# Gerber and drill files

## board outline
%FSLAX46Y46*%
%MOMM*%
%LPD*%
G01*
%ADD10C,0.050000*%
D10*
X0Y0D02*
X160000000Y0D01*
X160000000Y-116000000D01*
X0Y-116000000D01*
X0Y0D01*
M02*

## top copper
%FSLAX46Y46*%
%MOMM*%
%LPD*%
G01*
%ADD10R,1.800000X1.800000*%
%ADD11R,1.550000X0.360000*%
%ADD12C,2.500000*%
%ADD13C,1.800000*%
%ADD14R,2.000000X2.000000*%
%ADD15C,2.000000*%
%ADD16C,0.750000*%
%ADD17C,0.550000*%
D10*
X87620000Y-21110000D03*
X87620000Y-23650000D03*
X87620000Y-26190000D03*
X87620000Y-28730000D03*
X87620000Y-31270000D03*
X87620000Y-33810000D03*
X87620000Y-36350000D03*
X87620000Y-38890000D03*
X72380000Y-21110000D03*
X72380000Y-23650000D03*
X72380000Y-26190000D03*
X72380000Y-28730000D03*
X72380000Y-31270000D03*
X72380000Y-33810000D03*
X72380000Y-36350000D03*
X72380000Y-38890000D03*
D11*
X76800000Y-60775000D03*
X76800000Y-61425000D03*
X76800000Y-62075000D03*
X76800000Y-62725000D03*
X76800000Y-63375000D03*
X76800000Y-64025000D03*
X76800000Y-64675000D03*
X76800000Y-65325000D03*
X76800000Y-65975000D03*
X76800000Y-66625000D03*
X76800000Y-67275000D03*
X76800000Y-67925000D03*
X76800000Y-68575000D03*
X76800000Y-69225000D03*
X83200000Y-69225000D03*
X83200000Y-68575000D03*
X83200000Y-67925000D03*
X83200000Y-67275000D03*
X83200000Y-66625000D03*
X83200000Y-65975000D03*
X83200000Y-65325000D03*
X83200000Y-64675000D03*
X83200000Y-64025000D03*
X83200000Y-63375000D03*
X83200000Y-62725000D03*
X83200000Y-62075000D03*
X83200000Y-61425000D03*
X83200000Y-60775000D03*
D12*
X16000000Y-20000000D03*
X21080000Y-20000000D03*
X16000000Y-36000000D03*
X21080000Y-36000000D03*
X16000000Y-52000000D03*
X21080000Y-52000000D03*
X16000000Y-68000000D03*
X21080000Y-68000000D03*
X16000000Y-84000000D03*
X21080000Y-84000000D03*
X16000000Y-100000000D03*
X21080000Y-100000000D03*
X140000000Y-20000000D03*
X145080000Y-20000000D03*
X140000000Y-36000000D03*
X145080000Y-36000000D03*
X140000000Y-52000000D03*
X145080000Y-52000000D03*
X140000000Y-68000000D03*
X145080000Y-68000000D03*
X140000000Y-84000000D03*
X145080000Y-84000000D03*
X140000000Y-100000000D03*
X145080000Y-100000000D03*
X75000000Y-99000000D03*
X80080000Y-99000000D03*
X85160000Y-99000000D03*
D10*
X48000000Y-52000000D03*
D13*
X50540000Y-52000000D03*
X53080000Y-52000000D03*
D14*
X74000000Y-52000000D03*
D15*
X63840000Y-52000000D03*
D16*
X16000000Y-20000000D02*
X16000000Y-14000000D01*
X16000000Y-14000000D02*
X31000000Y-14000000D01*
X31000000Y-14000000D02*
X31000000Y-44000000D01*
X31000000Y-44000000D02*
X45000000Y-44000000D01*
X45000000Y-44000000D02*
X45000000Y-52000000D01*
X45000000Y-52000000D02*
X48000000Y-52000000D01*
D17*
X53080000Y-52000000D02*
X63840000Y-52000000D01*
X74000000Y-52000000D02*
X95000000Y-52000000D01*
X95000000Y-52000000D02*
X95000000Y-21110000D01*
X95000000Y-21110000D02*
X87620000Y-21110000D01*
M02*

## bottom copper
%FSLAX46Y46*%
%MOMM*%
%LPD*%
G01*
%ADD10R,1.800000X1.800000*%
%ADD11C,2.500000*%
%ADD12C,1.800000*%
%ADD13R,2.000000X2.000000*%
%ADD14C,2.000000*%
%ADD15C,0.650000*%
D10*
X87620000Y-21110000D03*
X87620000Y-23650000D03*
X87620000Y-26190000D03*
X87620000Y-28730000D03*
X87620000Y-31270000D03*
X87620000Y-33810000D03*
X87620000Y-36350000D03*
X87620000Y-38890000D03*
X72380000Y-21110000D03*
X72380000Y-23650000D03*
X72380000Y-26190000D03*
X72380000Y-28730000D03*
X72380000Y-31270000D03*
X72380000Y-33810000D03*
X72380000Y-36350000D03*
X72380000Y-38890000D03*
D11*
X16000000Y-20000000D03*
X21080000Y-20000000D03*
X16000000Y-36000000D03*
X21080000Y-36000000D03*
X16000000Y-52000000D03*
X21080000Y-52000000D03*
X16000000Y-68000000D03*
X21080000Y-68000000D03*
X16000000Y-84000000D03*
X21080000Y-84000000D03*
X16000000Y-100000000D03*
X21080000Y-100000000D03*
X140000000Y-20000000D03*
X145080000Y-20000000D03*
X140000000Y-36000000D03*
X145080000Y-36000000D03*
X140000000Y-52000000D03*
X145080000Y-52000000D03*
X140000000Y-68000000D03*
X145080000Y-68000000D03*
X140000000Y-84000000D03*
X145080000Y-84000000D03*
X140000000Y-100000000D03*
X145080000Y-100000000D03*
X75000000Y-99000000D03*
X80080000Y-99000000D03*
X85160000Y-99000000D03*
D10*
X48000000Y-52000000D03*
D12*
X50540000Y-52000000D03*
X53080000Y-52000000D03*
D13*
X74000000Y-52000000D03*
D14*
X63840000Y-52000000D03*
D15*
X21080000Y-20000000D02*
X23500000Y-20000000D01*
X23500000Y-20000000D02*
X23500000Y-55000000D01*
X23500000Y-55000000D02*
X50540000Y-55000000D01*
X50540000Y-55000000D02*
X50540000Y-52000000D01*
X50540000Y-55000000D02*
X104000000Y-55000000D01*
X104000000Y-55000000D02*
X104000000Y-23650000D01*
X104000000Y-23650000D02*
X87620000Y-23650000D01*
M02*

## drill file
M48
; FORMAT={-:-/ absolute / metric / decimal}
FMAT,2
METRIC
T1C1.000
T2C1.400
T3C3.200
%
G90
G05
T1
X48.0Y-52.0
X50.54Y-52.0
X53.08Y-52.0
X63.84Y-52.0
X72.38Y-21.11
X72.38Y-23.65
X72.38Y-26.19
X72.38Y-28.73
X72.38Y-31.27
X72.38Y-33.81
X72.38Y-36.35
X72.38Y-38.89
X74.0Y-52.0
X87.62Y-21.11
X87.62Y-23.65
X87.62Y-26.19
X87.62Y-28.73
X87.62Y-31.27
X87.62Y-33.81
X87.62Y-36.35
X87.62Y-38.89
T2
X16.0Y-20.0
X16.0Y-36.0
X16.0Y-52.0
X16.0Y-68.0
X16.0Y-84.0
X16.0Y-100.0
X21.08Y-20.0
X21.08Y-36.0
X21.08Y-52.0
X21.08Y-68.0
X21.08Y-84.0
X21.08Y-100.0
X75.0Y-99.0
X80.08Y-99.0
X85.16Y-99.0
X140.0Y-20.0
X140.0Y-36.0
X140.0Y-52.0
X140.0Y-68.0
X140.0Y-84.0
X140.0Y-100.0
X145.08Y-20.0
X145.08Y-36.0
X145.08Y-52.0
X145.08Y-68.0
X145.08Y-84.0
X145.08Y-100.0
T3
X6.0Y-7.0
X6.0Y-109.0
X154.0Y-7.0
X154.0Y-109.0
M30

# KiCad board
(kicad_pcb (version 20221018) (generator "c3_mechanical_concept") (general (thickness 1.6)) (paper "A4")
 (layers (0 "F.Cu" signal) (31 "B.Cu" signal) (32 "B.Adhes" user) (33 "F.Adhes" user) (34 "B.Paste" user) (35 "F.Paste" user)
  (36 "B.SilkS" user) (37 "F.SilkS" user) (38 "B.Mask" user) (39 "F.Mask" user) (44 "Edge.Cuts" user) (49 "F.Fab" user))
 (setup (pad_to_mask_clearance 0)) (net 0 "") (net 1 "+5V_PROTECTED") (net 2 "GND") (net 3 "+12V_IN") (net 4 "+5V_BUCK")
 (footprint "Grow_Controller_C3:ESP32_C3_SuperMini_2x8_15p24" (layer "F.Cu") (at 80 30)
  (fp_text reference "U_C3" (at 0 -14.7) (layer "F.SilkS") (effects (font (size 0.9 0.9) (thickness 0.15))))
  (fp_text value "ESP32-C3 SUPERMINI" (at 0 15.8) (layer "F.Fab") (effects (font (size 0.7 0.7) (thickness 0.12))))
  (pad "1" thru_hole rect (at 7.62 -8.89) (size 1.8 1.8) (drill 1.0) (layers "*.Cu" "*.Mask") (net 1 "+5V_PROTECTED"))
  (pad "2" thru_hole rect (at 7.62 -6.35) (size 1.8 1.8) (drill 1.0) (layers "*.Cu" "*.Mask") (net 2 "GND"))
  (pad "3" thru_hole rect (at 7.62 -3.81) (size 1.8 1.8) (drill 1.0) (layers "*.Cu" "*.Mask"))
  (pad "4" thru_hole rect (at 7.62 -1.27) (size 1.8 1.8) (drill 1.0) (layers "*.Cu" "*.Mask"))
  (pad "5" thru_hole rect (at 7.62 1.27) (size 1.8 1.8) (drill 1.0) (layers "*.Cu" "*.Mask"))
  (pad "6" thru_hole rect (at 7.62 3.81) (size 1.8 1.8) (drill 1.0) (layers "*.Cu" "*.Mask"))
  (pad "7" thru_hole rect (at 7.62 6.35) (size 1.8 1.8) (drill 1.0) (layers "*.Cu" "*.Mask"))
  (pad "8" thru_hole rect (at 7.62 8.89) (size 1.8 1.8) (drill 1.0) (layers "*.Cu" "*.Mask"))
  (pad "9" thru_hole rect (at -7.62 -8.89) (size 1.8 1.8) (drill 1.0) (layers "*.Cu" "*.Mask"))
  (pad "10" thru_hole rect (at -7.62 -6.35) (size 1.8 1.8) (drill 1.0) (layers "*.Cu" "*.Mask"))
  (pad "11" thru_hole rect (at -7.62 -3.81) (size 1.8 1.8) (drill 1.0) (layers "*.Cu" "*.Mask"))
  (pad "12" thru_hole rect (at -7.62 -1.27) (size 1.8 1.8) (drill 1.0) (layers "*.Cu" "*.Mask"))
  (pad "13" thru_hole rect (at -7.62 1.27) (size 1.8 1.8) (drill 1.0) (layers "*.Cu" "*.Mask"))
  (pad "14" thru_hole rect (at -7.62 3.81) (size 1.8 1.8) (drill 1.0) (layers "*.Cu" "*.Mask"))
  (pad "15" thru_hole rect (at -7.62 6.35) (size 1.8 1.8) (drill 1.0) (layers "*.Cu" "*.Mask"))
  (pad "16" thru_hole rect (at -7.62 8.89) (size 1.8 1.8) (drill 1.0) (layers "*.Cu" "*.Mask")))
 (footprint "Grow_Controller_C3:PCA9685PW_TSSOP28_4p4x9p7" (layer "F.Cu") (at 80 65)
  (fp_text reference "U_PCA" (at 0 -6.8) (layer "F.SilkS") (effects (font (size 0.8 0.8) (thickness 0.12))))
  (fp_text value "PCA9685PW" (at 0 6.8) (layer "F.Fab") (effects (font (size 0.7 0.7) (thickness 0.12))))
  (pad "1" smd rect (at -3.200 -4.225) (size 1.55 0.36) (layers "F.Cu" "F.Paste" "F.Mask"))
  (pad "2" smd rect (at -3.200 -3.575) (size 1.55 0.36) (layers "F.Cu" "F.Paste" "F.Mask"))
  (pad "3" smd rect (at -3.200 -2.925) (size 1.55 0.36) (layers "F.Cu" "F.Paste" "F.Mask"))
  (pad "4" smd rect (at -3.200 -2.275) (size 1.55 0.36) (layers "F.Cu" "F.Paste" "F.Mask"))
  (pad "5" smd rect (at -3.200 -1.625) (size 1.55 0.36) (layers "F.Cu" "F.Paste" "F.Mask"))
  (pad "6" smd rect (at -3.200 -0.975) (size 1.55 0.36) (layers "F.Cu" "F.Paste" "F.Mask"))
  (pad "7" smd rect (at -3.200 -0.325) (size 1.55 0.36) (layers "F.Cu" "F.Paste" "F.Mask"))
  (pad "8" smd rect (at -3.200 0.325) (size 1.55 0.36) (layers "F.Cu" "F.Paste" "F.Mask"))
  (pad "9" smd rect (at -3.200 0.975) (size 1.55 0.36) (layers "F.Cu" "F.Paste" "F.Mask"))
  (pad "10" smd rect (at -3.200 1.625) (size 1.55 0.36) (layers "F.Cu" "F.Paste" "F.Mask"))
  (pad "11" smd rect (at -3.200 2.275) (size 1.55 0.36) (layers "F.Cu" "F.Paste" "F.Mask"))
  (pad "12" smd rect (at -3.200 2.925) (size 1.55 0.36) (layers "F.Cu" "F.Paste" "F.Mask"))
  (pad "13" smd rect (at -3.200 3.575) (size 1.55 0.36) (layers "F.Cu" "F.Paste" "F.Mask"))
  (pad "14" smd rect (at -3.200 4.225) (size 1.55 0.36) (layers "F.Cu" "F.Paste" "F.Mask"))
  (pad "15" smd rect (at 3.200 4.225) (size 1.55 0.36) (layers "F.Cu" "F.Paste" "F.Mask"))
  (pad "16" smd rect (at 3.200 3.575) (size 1.55 0.36) (layers "F.Cu" "F.Paste" "F.Mask"))
  (pad "17" smd rect (at 3.200 2.925) (size 1.55 0.36) (layers "F.Cu" "F.Paste" "F.Mask"))
  (pad "18" smd rect (at 3.200 2.275) (size 1.55 0.36) (layers "F.Cu" "F.Paste" "F.Mask"))
  (pad "19" smd rect (at 3.200 1.625) (size 1.55 0.36) (layers "F.Cu" "F.Paste" "F.Mask"))
  (pad "20" smd rect (at 3.200 0.975) (size 1.55 0.36) (layers "F.Cu" "F.Paste" "F.Mask"))
  (pad "21" smd rect (at 3.200 0.325) (size 1.55 0.36) (layers "F.Cu" "F.Paste" "F.Mask"))
  (pad "22" smd rect (at 3.200 -0.325) (size 1.55 0.36) (layers "F.Cu" "F.Paste" "F.Mask"))
  (pad "23" smd rect (at 3.200 -0.975) (size 1.55 0.36) (layers "F.Cu" "F.Paste" "F.Mask"))
  (pad "24" smd rect (at 3.200 -1.625) (size 1.55 0.36) (layers "F.Cu" "F.Paste" "F.Mask"))
  (pad "25" smd rect (at 3.200 -2.275) (size 1.55 0.36) (layers "F.Cu" "F.Paste" "F.Mask"))
  (pad "26" smd rect (at 3.200 -2.925) (size 1.55 0.36) (layers "F.Cu" "F.Paste" "F.Mask"))
  (pad "27" smd rect (at 3.200 -3.575) (size 1.55 0.36) (layers "F.Cu" "F.Paste" "F.Mask"))
  (pad "28" smd rect (at 3.200 -4.225) (size 1.55 0.36) (layers "F.Cu" "F.Paste" "F.Mask")))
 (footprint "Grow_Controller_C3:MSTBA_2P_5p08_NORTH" (layer "F.Cu") (at 16 20)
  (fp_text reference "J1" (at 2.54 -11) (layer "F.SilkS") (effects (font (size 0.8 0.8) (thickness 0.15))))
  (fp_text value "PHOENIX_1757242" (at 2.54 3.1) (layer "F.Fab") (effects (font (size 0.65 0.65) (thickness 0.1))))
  (pad "1" thru_hole circle (at 0.00 0) (size 2.5 2.5) (drill 1.4) (layers "*.Cu" "*.Mask") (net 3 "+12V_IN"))
  (pad "2" thru_hole circle (at 5.08 0) (size 2.5 2.5) (drill 1.4) (layers "*.Cu" "*.Mask") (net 2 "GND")))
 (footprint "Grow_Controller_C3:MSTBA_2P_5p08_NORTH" (layer "F.Cu") (at 16 36)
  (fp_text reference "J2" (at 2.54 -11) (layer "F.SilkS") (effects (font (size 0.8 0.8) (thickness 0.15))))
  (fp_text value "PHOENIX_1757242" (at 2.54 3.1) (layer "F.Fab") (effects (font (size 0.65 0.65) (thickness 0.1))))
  (pad "1" thru_hole circle (at 0.00 0) (size 2.5 2.5) (drill 1.4) (layers "*.Cu" "*.Mask"))
  (pad "2" thru_hole circle (at 5.08 0) (size 2.5 2.5) (drill 1.4) (layers "*.Cu" "*.Mask")))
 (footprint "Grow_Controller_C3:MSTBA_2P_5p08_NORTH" (layer "F.Cu") (at 16 52)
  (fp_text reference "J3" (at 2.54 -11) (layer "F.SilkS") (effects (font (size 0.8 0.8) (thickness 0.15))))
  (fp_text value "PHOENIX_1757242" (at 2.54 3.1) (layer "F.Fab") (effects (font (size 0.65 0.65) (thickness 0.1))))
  (pad "1" thru_hole circle (at 0.00 0) (size 2.5 2.5) (drill 1.4) (layers "*.Cu" "*.Mask"))
  (pad "2" thru_hole circle (at 5.08 0) (size 2.5 2.5) (drill 1.4) (layers "*.Cu" "*.Mask")))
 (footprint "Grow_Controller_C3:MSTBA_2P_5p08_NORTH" (layer "F.Cu") (at 16 68)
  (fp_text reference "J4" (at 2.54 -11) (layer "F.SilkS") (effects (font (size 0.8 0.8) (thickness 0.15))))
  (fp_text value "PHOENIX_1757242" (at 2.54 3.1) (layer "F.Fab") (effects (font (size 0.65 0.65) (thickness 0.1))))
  (pad "1" thru_hole circle (at 0.00 0) (size 2.5 2.5) (drill 1.4) (layers "*.Cu" "*.Mask"))
  (pad "2" thru_hole circle (at 5.08 0) (size 2.5 2.5) (drill 1.4) (layers "*.Cu" "*.Mask")))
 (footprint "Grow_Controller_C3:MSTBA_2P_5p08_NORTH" (layer "F.Cu") (at 16 84)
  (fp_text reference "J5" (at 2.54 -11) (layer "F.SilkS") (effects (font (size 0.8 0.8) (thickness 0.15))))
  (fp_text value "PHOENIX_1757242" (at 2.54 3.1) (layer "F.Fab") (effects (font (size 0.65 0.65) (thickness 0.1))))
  (pad "1" thru_hole circle (at 0.00 0) (size 2.5 2.5) (drill 1.4) (layers "*.Cu" "*.Mask"))
  (pad "2" thru_hole circle (at 5.08 0) (size 2.5 2.5) (drill 1.4) (layers "*.Cu" "*.Mask")))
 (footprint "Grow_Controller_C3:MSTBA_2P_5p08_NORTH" (layer "F.Cu") (at 16 100)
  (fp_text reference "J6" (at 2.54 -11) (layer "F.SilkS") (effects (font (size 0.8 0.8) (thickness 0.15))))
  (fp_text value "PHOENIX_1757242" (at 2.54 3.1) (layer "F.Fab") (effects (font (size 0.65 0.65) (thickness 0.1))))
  (pad "1" thru_hole circle (at 0.00 0) (size 2.5 2.5) (drill 1.4) (layers "*.Cu" "*.Mask"))
  (pad "2" thru_hole circle (at 5.08 0) (size 2.5 2.5) (drill 1.4) (layers "*.Cu" "*.Mask")))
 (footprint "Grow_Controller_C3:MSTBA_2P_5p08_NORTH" (layer "F.Cu") (at 140 20)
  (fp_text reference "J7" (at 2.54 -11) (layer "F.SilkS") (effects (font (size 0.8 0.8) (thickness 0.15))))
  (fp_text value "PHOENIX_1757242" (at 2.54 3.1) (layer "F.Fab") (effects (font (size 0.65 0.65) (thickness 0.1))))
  (pad "1" thru_hole circle (at 0.00 0) (size 2.5 2.5) (drill 1.4) (layers "*.Cu" "*.Mask"))
  (pad "2" thru_hole circle (at 5.08 0) (size 2.5 2.5) (drill 1.4) (layers "*.Cu" "*.Mask")))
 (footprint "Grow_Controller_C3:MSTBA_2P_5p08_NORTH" (layer "F.Cu") (at 140 36)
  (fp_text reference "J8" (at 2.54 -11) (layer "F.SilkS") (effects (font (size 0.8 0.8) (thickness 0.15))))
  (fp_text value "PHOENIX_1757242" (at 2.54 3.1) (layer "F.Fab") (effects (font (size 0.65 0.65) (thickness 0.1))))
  (pad "1" thru_hole circle (at 0.00 0) (size 2.5 2.5) (drill 1.4) (layers "*.Cu" "*.Mask"))
  (pad "2" thru_hole circle (at 5.08 0) (size 2.5 2.5) (drill 1.4) (layers "*.Cu" "*.Mask")))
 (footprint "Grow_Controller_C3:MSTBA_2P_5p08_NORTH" (layer "F.Cu") (at 140 52)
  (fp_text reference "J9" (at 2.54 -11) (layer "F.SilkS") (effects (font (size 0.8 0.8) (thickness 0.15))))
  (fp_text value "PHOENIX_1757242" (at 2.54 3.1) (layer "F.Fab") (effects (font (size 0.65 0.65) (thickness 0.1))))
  (pad "1" thru_hole circle (at 0.00 0) (size 2.5 2.5) (drill 1.4) (layers "*.Cu" "*.Mask"))
  (pad "2" thru_hole circle (at 5.08 0) (size 2.5 2.5) (drill 1.4) (layers "*.Cu" "*.Mask")))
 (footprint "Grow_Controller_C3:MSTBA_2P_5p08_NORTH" (layer "F.Cu") (at 140 68)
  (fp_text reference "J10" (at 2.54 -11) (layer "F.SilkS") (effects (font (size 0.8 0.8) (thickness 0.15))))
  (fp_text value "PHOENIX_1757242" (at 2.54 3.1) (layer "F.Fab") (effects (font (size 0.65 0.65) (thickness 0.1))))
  (pad "1" thru_hole circle (at 0.00 0) (size 2.5 2.5) (drill 1.4) (layers "*.Cu" "*.Mask"))
  (pad "2" thru_hole circle (at 5.08 0) (size 2.5 2.5) (drill 1.4) (layers "*.Cu" "*.Mask")))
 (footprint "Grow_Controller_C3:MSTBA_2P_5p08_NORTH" (layer "F.Cu") (at 140 84)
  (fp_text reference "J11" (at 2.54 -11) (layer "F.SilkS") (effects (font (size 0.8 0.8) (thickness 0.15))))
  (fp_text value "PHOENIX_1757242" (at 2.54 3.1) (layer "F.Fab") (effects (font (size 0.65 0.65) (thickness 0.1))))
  (pad "1" thru_hole circle (at 0.00 0) (size 2.5 2.5) (drill 1.4) (layers "*.Cu" "*.Mask"))
  (pad "2" thru_hole circle (at 5.08 0) (size 2.5 2.5) (drill 1.4) (layers "*.Cu" "*.Mask")))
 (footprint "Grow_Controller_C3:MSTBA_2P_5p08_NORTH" (layer "F.Cu") (at 140 100)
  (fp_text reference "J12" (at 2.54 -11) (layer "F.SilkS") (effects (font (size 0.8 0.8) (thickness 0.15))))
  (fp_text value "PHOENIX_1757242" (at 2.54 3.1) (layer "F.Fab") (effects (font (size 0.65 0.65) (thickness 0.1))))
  (pad "1" thru_hole circle (at 0.00 0) (size 2.5 2.5) (drill 1.4) (layers "*.Cu" "*.Mask"))
  (pad "2" thru_hole circle (at 5.08 0) (size 2.5 2.5) (drill 1.4) (layers "*.Cu" "*.Mask")))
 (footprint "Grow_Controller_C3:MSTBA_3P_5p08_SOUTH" (layer "F.Cu") (at 75 99)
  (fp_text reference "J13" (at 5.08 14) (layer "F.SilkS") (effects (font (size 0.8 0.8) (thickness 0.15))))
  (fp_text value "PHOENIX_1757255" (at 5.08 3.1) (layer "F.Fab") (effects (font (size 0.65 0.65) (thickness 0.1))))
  (pad "1" thru_hole circle (at 0.00 0) (size 2.5 2.5) (drill 1.4) (layers "*.Cu" "*.Mask"))
  (pad "2" thru_hole circle (at 5.08 0) (size 2.5 2.5) (drill 1.4) (layers "*.Cu" "*.Mask"))
  (pad "3" thru_hole circle (at 10.16 0) (size 2.5 2.5) (drill 1.4) (layers "*.Cu" "*.Mask")))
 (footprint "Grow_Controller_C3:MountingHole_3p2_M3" (layer "F.Cu") (at 6 7)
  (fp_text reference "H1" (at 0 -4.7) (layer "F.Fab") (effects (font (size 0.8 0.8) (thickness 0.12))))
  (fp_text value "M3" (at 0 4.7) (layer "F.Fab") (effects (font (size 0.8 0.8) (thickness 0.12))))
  (pad "" np_thru_hole circle (at 0 0) (size 3.2 3.2) (drill 3.2) (layers "*.Cu" "*.Mask")))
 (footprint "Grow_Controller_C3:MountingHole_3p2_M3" (layer "F.Cu") (at 154 7)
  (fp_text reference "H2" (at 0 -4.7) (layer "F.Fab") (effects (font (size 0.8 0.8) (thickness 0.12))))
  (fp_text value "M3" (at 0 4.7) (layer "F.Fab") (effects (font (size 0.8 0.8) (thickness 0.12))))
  (pad "" np_thru_hole circle (at 0 0) (size 3.2 3.2) (drill 3.2) (layers "*.Cu" "*.Mask")))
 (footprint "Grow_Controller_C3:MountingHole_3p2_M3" (layer "F.Cu") (at 6 109)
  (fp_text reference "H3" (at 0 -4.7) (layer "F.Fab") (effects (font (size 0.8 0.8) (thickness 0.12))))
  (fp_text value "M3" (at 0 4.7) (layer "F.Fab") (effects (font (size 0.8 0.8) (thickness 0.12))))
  (pad "" np_thru_hole circle (at 0 0) (size 3.2 3.2) (drill 3.2) (layers "*.Cu" "*.Mask")))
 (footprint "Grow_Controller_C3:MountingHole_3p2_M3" (layer "F.Cu") (at 154 109)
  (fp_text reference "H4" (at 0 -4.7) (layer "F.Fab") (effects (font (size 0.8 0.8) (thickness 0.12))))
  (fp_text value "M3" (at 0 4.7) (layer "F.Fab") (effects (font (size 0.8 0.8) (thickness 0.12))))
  (pad "" np_thru_hole circle (at 0 0) (size 3.2 3.2) (drill 3.2) (layers "*.Cu" "*.Mask")))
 (gr_rect (start 0 0) (end 160 116) (stroke (width 0.05) (type default)) (fill none) (layer "Edge.Cuts"))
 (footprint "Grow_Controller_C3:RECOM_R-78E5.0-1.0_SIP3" (layer "F.Cu") (at 48 52)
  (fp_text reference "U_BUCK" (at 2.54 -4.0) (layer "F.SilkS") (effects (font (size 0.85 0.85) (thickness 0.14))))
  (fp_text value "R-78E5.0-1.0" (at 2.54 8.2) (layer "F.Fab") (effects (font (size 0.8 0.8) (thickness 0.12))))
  (pad "1" thru_hole rect (at 0 0) (size 1.8 1.8) (drill 1.0) (layers "*.Cu" "*.Mask") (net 3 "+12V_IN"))
  (pad "2" thru_hole circle (at 2.54 0) (size 1.8 1.8) (drill 1.0) (layers "*.Cu" "*.Mask") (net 2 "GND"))
  (pad "3" thru_hole circle (at 5.08 0) (size 1.8 1.8) (drill 1.0) (layers "*.Cu" "*.Mask") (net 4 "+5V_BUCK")))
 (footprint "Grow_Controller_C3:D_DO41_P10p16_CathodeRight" (layer "F.Cu") (at 63.84 52)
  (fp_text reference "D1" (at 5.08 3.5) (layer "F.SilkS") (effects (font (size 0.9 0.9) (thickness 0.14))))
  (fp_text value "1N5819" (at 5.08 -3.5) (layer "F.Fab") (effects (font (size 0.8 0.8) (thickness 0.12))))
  (pad "1" thru_hole rect (at 10.16 0) (size 2.0 2.0) (drill 1.0) (layers "*.Cu" "*.Mask") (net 1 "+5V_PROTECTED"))
  (pad "2" thru_hole circle (at 0 0) (size 2.0 2.0) (drill 1.0) (layers "*.Cu" "*.Mask") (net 4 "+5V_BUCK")))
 (segment (start 16 20) (end 16 14) (width 0.75) (layer "F.Cu") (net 3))
 (segment (start 16 14) (end 31 14) (width 0.75) (layer "F.Cu") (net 3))
 (segment (start 31 14) (end 31 44) (width 0.75) (layer "F.Cu") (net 3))
 (segment (start 31 44) (end 45 44) (width 0.75) (layer "F.Cu") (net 3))
 (segment (start 45 44) (end 45 52) (width 0.75) (layer "F.Cu") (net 3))
 (segment (start 45 52) (end 48 52) (width 0.75) (layer "F.Cu") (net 3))
 (segment (start 21.08 20) (end 23.5 20) (width 0.65) (layer "B.Cu") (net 2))
 (segment (start 23.5 20) (end 23.5 55) (width 0.65) (layer "B.Cu") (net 2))
 (segment (start 23.5 55) (end 50.54 55) (width 0.65) (layer "B.Cu") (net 2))
 (segment (start 50.54 55) (end 50.54 52) (width 0.65) (layer "B.Cu") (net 2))
 (segment (start 50.54 55) (end 104 55) (width 0.65) (layer "B.Cu") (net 2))
 (segment (start 104 55) (end 104 23.65) (width 0.65) (layer "B.Cu") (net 2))
 (segment (start 104 23.65) (end 87.62 23.65) (width 0.65) (layer "B.Cu") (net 2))
 (segment (start 53.08 52) (end 63.84 52) (width 0.55) (layer "F.Cu") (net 4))
 (segment (start 74 52) (end 95 52) (width 0.55) (layer "F.Cu") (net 1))
 (segment (start 95 52) (end 95 21.11) (width 0.55) (layer "F.Cu") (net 1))
 (segment (start 95 21.11) (end 87.62 21.11) (width 0.55) (layer "F.Cu") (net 1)))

